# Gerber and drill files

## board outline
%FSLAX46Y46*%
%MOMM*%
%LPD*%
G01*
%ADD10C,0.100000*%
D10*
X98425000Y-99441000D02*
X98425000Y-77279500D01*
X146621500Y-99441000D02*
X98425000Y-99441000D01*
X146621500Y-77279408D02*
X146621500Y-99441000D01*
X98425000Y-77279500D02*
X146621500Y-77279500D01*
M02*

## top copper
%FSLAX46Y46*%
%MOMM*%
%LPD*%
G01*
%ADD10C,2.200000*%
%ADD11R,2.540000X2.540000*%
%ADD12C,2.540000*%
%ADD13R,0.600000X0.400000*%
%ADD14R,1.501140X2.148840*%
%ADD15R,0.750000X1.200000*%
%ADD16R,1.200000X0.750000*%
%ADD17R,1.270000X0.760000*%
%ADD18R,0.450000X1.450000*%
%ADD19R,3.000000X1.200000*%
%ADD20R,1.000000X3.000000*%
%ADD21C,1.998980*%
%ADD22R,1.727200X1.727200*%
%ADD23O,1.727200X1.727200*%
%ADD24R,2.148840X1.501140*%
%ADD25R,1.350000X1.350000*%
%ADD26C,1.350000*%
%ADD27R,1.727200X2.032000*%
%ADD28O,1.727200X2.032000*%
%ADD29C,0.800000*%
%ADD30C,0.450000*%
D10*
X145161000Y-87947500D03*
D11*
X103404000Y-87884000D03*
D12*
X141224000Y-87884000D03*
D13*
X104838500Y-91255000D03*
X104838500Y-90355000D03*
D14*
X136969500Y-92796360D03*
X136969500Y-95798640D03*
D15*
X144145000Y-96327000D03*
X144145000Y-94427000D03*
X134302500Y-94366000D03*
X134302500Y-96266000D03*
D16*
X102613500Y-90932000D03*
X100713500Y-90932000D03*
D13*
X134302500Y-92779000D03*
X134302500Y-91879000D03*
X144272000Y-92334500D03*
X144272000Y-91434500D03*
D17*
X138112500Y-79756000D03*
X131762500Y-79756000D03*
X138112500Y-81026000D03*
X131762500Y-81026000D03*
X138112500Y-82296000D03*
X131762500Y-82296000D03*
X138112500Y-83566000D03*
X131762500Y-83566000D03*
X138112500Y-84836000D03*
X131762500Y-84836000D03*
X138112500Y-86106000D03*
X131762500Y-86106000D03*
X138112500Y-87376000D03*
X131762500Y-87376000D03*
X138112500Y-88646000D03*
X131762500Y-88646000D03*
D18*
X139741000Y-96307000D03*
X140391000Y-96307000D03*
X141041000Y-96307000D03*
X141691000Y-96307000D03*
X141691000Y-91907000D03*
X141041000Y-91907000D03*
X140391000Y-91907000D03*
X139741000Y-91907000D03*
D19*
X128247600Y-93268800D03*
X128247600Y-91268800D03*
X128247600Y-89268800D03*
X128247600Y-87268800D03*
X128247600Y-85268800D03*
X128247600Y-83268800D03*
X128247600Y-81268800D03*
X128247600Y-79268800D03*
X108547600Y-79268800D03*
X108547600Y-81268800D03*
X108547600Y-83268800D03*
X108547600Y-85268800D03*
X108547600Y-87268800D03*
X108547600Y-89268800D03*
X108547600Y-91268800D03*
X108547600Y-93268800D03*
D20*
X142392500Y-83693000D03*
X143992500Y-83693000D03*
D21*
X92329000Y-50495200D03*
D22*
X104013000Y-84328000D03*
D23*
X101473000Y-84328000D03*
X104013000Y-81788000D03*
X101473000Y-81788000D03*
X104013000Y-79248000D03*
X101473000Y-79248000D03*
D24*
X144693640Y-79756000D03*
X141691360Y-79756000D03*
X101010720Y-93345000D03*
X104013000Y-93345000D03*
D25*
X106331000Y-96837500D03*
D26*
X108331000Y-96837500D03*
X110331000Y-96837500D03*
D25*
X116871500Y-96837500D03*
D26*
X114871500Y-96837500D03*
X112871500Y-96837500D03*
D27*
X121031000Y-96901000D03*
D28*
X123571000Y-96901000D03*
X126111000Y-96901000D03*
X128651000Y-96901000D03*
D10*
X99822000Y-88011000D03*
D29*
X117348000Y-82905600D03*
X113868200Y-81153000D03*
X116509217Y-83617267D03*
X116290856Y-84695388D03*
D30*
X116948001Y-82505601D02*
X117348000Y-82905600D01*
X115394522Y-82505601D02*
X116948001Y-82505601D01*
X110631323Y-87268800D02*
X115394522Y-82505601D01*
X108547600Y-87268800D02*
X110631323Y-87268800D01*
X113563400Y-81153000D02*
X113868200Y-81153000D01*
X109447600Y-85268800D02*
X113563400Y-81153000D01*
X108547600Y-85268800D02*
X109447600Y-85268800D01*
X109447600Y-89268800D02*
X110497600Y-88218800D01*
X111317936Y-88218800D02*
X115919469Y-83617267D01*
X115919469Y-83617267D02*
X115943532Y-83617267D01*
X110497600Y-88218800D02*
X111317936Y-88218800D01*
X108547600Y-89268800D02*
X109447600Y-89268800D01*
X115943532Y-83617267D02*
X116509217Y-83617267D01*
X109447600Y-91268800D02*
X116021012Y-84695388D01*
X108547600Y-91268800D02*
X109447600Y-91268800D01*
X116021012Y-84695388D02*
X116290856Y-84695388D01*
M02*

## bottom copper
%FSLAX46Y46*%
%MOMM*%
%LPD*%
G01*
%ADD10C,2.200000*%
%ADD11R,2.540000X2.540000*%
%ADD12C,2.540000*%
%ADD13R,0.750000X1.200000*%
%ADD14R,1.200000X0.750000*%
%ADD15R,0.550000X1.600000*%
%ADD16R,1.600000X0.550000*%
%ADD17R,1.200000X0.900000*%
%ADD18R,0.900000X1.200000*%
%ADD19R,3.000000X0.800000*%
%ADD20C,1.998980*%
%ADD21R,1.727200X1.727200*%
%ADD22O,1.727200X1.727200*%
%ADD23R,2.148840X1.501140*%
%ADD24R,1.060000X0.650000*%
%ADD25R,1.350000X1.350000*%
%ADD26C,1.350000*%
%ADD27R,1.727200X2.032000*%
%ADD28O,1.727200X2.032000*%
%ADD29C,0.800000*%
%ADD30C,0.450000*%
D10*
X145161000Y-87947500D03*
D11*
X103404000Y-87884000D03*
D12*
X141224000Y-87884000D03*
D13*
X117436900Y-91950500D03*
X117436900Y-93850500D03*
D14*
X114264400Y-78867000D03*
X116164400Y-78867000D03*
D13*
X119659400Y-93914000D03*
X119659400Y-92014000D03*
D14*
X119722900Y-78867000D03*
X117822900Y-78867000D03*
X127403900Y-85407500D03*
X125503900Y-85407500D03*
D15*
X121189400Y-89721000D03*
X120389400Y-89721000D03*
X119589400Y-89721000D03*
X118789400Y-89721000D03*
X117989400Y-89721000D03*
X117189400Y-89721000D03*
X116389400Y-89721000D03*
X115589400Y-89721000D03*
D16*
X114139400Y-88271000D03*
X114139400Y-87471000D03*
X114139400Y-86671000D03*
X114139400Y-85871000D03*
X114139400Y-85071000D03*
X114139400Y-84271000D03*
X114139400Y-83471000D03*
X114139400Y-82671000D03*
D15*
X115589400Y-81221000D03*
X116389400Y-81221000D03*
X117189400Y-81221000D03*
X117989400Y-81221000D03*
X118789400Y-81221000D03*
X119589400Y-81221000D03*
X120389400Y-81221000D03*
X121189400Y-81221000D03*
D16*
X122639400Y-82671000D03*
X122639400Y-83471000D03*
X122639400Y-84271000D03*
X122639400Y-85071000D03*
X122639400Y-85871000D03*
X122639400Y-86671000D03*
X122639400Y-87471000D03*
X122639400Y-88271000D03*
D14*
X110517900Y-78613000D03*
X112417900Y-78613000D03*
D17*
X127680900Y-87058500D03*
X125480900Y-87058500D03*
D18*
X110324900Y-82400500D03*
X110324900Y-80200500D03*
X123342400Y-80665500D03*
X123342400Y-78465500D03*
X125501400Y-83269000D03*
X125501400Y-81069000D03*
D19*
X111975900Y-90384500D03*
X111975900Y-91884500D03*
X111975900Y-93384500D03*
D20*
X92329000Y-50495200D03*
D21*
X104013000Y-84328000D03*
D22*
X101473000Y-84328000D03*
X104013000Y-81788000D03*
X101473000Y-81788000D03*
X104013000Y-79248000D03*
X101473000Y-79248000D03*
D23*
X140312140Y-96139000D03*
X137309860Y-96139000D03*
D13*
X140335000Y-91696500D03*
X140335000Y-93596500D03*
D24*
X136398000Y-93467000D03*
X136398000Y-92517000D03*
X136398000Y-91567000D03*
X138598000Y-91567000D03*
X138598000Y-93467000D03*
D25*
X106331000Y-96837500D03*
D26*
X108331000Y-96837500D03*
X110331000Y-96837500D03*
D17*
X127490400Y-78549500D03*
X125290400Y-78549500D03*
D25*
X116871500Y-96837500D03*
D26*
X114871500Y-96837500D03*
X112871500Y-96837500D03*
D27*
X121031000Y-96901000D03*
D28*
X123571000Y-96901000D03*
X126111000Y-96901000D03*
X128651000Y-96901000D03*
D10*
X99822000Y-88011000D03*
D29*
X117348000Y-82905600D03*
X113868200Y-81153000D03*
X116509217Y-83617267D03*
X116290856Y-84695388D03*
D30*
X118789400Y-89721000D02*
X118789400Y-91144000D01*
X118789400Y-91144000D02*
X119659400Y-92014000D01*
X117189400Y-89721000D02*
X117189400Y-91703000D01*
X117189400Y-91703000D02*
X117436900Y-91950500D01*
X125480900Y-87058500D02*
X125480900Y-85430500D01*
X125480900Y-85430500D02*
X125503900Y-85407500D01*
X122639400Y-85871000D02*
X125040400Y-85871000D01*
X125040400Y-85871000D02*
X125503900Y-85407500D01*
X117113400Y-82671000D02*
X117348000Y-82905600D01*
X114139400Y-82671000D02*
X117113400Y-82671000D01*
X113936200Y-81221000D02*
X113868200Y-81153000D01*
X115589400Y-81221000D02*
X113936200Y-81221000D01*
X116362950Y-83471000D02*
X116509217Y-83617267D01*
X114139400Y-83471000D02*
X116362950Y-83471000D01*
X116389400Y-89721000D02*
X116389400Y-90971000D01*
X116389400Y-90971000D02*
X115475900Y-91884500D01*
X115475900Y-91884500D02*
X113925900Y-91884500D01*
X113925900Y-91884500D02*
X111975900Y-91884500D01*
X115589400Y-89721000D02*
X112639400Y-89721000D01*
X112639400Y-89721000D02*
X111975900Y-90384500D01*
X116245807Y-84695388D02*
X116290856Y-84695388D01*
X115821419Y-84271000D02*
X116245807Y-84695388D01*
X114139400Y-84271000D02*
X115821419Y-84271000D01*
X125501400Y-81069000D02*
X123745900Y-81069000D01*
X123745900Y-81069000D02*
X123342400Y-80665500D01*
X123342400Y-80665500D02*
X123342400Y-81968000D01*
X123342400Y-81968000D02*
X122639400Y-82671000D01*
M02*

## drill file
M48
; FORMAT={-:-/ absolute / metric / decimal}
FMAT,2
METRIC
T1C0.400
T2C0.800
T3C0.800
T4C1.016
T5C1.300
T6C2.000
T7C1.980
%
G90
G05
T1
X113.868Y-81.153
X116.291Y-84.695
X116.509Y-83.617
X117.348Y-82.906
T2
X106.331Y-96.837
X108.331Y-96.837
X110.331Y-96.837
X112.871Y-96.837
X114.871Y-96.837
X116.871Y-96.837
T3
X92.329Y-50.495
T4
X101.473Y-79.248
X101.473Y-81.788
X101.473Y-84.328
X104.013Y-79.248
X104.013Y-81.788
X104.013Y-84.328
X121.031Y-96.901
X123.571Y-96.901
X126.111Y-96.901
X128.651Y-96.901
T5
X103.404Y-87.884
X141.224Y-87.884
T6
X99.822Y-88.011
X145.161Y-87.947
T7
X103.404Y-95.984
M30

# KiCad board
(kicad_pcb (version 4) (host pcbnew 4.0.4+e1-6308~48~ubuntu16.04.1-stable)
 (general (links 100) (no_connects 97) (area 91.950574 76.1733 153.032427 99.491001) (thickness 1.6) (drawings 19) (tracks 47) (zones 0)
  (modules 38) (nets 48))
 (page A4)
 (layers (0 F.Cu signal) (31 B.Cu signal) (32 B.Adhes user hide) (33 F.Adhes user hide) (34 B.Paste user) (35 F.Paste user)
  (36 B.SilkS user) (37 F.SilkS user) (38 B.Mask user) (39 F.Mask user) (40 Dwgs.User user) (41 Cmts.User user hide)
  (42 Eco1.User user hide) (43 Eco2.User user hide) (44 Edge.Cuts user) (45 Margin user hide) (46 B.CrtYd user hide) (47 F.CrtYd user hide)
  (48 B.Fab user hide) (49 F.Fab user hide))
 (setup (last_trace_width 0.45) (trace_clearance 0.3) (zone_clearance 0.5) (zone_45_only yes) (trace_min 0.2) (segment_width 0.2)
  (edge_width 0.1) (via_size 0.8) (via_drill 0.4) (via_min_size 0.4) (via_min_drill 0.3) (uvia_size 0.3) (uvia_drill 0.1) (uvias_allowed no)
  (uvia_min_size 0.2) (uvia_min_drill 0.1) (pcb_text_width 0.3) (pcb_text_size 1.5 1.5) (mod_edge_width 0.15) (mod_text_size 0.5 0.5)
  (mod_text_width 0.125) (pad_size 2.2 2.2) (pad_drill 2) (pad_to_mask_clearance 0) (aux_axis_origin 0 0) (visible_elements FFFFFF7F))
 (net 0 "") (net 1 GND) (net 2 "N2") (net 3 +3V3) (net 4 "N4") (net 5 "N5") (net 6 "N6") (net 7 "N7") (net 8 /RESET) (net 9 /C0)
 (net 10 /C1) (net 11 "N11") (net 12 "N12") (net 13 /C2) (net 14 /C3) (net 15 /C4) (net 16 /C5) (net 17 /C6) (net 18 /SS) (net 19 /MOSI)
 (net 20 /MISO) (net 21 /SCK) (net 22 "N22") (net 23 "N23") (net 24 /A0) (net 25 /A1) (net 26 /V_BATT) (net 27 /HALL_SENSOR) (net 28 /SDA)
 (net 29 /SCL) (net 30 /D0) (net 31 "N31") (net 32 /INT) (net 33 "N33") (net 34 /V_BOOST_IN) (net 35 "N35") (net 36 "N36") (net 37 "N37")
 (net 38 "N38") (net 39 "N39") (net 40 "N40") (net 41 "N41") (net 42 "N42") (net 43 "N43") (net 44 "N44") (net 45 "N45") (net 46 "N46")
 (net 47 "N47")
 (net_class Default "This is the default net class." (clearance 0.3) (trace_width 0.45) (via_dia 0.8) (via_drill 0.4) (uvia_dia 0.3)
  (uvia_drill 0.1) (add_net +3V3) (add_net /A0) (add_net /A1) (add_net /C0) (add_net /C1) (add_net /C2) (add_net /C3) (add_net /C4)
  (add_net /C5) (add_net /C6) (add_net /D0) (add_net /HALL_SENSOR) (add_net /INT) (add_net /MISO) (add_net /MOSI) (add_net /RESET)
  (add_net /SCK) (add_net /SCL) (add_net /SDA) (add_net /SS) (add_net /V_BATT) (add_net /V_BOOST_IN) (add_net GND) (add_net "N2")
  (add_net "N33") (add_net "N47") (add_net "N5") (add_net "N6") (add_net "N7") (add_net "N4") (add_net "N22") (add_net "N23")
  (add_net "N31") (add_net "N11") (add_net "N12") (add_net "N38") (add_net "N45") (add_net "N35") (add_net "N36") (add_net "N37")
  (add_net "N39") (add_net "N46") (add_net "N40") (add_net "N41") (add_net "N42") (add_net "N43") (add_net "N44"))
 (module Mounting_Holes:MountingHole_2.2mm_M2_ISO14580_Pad (layer F.Cu) (at 145.161 87.9475)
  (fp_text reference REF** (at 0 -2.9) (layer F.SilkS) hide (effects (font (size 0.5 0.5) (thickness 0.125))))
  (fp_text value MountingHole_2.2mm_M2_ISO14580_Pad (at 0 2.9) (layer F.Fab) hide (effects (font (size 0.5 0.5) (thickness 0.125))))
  (pad "" thru_hole circle (at 0 0) (size 2.2 2.2) (drill 2) (layers *.Cu *.Mask F.SilkS) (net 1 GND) (zone_connect 2)))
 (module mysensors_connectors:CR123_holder (layer B.Cu) (at 103.404 87.884 270)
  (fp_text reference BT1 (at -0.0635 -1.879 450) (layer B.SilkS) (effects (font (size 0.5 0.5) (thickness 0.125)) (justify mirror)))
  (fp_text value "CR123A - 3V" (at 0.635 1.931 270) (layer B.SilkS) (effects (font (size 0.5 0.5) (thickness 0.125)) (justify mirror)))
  (pad 1 thru_hole rect (at 0 0 270) (size 2.54 2.54) (drill 1.3) (layers *.Cu *.Mask B.SilkS) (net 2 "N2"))
  (pad 2 thru_hole circle (at 0 -37.82 270) (size 2.54 2.54) (drill 1.3) (layers *.Cu *.Mask B.SilkS) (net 1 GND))
  (pad "" np_thru_hole circle (at 8.1 0 270) (size 1.98 1.98) (drill 1.98) (layers *.Cu Dwgs.User)))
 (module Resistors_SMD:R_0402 (layer F.Cu) (at 104.8385 90.805 90)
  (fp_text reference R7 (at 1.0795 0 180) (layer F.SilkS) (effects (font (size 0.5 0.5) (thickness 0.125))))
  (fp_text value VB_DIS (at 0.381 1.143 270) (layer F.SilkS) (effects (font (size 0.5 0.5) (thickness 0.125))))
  (pad 1 smd rect (at -0.45 0 90) (size 0.4 0.6) (layers F.Cu F.Paste F.Mask) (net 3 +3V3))
  (pad 2 smd rect (at 0.45 0 90) (size 0.4 0.6) (layers F.Cu F.Paste F.Mask) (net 2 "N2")))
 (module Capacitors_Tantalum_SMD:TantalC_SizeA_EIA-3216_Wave (layer F.Cu) (at 136.9695 94.2975 90)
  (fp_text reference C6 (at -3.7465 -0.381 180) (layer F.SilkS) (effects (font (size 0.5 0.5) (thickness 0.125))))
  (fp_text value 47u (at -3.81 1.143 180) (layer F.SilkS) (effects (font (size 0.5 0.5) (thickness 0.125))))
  (pad 2 smd rect (at 1.50114 0 90) (size 2.14884 1.50114) (layers F.Cu F.Paste F.Mask) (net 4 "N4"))
  (pad 1 smd rect (at -1.50114 0 90) (size 2.14884 1.50114) (layers F.Cu F.Paste F.Mask) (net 1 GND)))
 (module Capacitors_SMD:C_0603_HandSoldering (layer B.Cu) (at 117.4369 92.9005 270)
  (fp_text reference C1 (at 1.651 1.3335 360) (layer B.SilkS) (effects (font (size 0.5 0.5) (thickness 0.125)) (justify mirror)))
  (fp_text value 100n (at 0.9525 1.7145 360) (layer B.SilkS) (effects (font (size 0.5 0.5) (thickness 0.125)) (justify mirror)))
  (pad 1 smd rect (at -0.95 0 270) (size 1.2 0.75) (layers B.Cu B.Paste B.Mask) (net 3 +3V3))
  (pad 2 smd rect (at 0.95 0 270) (size 1.2 0.75) (layers B.Cu B.Paste B.Mask) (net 1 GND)))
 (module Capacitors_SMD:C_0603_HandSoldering (layer B.Cu) (at 115.2144 78.867)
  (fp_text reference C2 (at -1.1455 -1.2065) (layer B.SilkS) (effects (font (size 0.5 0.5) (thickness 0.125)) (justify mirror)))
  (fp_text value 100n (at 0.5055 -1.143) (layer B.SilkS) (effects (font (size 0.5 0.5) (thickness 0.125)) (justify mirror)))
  (pad 1 smd rect (at -0.95 0) (size 1.2 0.75) (layers B.Cu B.Paste B.Mask) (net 1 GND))
  (pad 2 smd rect (at 0.95 0) (size 1.2 0.75) (layers B.Cu B.Paste B.Mask) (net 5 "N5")))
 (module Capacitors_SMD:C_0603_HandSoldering (layer B.Cu) (at 119.6594 92.964 90)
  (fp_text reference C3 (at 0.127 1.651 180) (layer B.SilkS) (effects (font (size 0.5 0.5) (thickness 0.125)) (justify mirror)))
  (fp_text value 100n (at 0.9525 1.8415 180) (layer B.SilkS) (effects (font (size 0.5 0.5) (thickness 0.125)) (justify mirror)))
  (pad 1 smd rect (at -0.95 0 90) (size 1.2 0.75) (layers B.Cu B.Paste B.Mask) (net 1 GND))
  (pad 2 smd rect (at 0.95 0 90) (size 1.2 0.75) (layers B.Cu B.Paste B.Mask) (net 3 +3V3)))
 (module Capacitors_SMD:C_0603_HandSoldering (layer B.Cu) (at 118.7729 78.867 180)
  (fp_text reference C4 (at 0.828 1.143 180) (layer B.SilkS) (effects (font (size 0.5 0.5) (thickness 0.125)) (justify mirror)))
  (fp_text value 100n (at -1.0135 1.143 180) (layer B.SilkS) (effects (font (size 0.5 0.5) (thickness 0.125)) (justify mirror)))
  (pad 1 smd rect (at -0.95 0 180) (size 1.2 0.75) (layers B.Cu B.Paste B.Mask) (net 1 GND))
  (pad 2 smd rect (at 0.95 0 180) (size 1.2 0.75) (layers B.Cu B.Paste B.Mask) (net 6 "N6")))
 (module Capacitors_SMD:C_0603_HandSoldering (layer F.Cu) (at 144.145 95.377 90)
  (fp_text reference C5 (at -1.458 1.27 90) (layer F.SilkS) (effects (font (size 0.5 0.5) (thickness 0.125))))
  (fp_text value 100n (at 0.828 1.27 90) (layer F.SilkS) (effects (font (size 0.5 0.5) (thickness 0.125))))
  (pad 1 smd rect (at -0.95 0 90) (size 1.2 0.75) (layers F.Cu F.Paste F.Mask) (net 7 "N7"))
  (pad 2 smd rect (at 0.95 0 90) (size 1.2 0.75) (layers F.Cu F.Paste F.Mask) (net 1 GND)))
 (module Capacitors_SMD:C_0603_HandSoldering (layer B.Cu) (at 126.4539 85.4075 180)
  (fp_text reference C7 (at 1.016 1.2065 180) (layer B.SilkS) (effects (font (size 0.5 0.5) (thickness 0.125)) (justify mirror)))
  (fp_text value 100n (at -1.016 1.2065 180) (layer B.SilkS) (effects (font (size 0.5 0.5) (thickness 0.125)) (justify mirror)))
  (pad 1 smd rect (at -0.95 0 180) (size 1.2 0.75) (layers B.Cu B.Paste B.Mask) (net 1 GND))
  (pad 2 smd rect (at 0.95 0 180) (size 1.2 0.75) (layers B.Cu B.Paste B.Mask) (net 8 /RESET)))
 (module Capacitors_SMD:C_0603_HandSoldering (layer F.Cu) (at 134.3025 95.316 270)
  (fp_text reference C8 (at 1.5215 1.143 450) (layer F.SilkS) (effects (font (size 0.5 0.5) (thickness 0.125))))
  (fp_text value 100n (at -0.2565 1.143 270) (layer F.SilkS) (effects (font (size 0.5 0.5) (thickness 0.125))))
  (pad 1 smd rect (at -0.95 0 270) (size 1.2 0.75) (layers F.Cu F.Paste F.Mask) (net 4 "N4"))
  (pad 2 smd rect (at 0.95 0 270) (size 1.2 0.75) (layers F.Cu F.Paste F.Mask) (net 1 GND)))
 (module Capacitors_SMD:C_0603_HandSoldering (layer F.Cu) (at 101.6635 90.932 180)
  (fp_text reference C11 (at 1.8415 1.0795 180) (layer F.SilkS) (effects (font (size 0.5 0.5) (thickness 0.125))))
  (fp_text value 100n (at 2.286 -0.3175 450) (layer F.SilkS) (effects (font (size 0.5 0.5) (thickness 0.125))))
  (pad 1 smd rect (at -0.95 0 180) (size 1.2 0.75) (layers F.Cu F.Paste F.Mask) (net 3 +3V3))
  (pad 2 smd rect (at 0.95 0 180) (size 1.2 0.75) (layers F.Cu F.Paste F.Mask) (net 1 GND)))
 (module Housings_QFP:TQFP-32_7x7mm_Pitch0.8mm (layer B.Cu) (at 118.3894 85.471 90)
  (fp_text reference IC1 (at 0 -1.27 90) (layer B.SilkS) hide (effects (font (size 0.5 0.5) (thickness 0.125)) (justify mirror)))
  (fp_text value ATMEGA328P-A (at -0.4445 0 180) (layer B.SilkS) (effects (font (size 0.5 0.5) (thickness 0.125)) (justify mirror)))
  (pad 1 smd rect (at -4.25 2.8 90) (size 1.6 0.55) (layers B.Cu B.Paste B.Mask) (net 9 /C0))
  (pad 2 smd rect (at -4.25 2 90) (size 1.6 0.55) (layers B.Cu B.Paste B.Mask) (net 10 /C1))
  (pad 3 smd rect (at -4.25 1.2 90) (size 1.6 0.55) (layers B.Cu B.Paste B.Mask) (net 1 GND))
  (pad 4 smd rect (at -4.25 0.4 90) (size 1.6 0.55) (layers B.Cu B.Paste B.Mask) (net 3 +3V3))
  (pad 5 smd rect (at -4.25 -0.4 90) (size 1.6 0.55) (layers B.Cu B.Paste B.Mask) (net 1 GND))
  (pad 6 smd rect (at -4.25 -1.2 90) (size 1.6 0.55) (layers B.Cu B.Paste B.Mask) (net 3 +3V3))
  (pad 7 smd rect (at -4.25 -2 90) (size 1.6 0.55) (layers B.Cu B.Paste B.Mask) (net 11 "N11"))
  (pad 8 smd rect (at -4.25 -2.8 90) (size 1.6 0.55) (layers B.Cu B.Paste B.Mask) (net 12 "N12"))
  (pad 9 smd rect (at -2.8 -4.25) (size 1.6 0.55) (layers B.Cu B.Paste B.Mask) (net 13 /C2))
  (pad 10 smd rect (at -2 -4.25) (size 1.6 0.55) (layers B.Cu B.Paste B.Mask) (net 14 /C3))
  (pad 11 smd rect (at -1.2 -4.25) (size 1.6 0.55) (layers B.Cu B.Paste B.Mask) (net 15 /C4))
  (pad 12 smd rect (at -0.4 -4.25) (size 1.6 0.55) (layers B.Cu B.Paste B.Mask) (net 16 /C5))
  (pad 13 smd rect (at 0.4 -4.25) (size 1.6 0.55) (layers B.Cu B.Paste B.Mask) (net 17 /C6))
  (pad 14 smd rect (at 1.2 -4.25) (size 1.6 0.55) (layers B.Cu B.Paste B.Mask) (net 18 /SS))
  (pad 15 smd rect (at 2 -4.25) (size 1.6 0.55) (layers B.Cu B.Paste B.Mask) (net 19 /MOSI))
  (pad 16 smd rect (at 2.8 -4.25) (size 1.6 0.55) (layers B.Cu B.Paste B.Mask) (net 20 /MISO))
  (pad 17 smd rect (at 4.25 -2.8 90) (size 1.6 0.55) (layers B.Cu B.Paste B.Mask) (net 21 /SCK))
  (pad 18 smd rect (at 4.25 -2 90) (size 1.6 0.55) (layers B.Cu B.Paste B.Mask) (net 5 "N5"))
  (pad 19 smd rect (at 4.25 -1.2 90) (size 1.6 0.55) (layers B.Cu B.Paste B.Mask) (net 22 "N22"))
  (pad 20 smd rect (at 4.25 -0.4 90) (size 1.6 0.55) (layers B.Cu B.Paste B.Mask) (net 6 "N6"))
  (pad 21 smd rect (at 4.25 0.4 90) (size 1.6 0.55) (layers B.Cu B.Paste B.Mask) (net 1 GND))
  (pad 22 smd rect (at 4.25 1.2 90) (size 1.6 0.55) (layers B.Cu B.Paste B.Mask) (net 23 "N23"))
  (pad 23 smd rect (at 4.25 2 90) (size 1.6 0.55) (layers B.Cu B.Paste B.Mask) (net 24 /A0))
  (pad 24 smd rect (at 4.25 2.8 90) (size 1.6 0.55) (layers B.Cu B.Paste B.Mask) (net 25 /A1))
  (pad 25 smd rect (at 2.8 4.25) (size 1.6 0.55) (layers B.Cu B.Paste B.Mask) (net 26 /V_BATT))
  (pad 26 smd rect (at 2 4.25) (size 1.6 0.55) (layers B.Cu B.Paste B.Mask) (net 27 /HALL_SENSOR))
  (pad 27 smd rect (at 1.2 4.25) (size 1.6 0.55) (layers B.Cu B.Paste B.Mask) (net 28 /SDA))
  (pad 28 smd rect (at 0.4 4.25) (size 1.6 0.55) (layers B.Cu B.Paste B.Mask) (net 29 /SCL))
  (pad 29 smd rect (at -0.4 4.25) (size 1.6 0.55) (layers B.Cu B.Paste B.Mask) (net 8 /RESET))
  (pad 30 smd rect (at -1.2 4.25) (size 1.6 0.55) (layers B.Cu B.Paste B.Mask) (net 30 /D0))
  (pad 31 smd rect (at -2 4.25) (size 1.6 0.55) (layers B.Cu B.Paste B.Mask) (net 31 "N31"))
  (pad 32 smd rect (at -2.8 4.25) (size 1.6 0.55) (layers B.Cu B.Paste B.Mask) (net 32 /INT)))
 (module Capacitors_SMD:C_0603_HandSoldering (layer B.Cu) (at 111.4679 78.613)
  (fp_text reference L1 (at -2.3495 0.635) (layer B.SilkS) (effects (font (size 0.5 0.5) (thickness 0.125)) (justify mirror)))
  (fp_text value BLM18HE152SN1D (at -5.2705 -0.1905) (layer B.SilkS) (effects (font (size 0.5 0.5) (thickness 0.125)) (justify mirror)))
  (pad 1 smd rect (at -0.95 0) (size 1.2 0.75) (layers B.Cu B.Paste B.Mask) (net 3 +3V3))
  (pad 2 smd rect (at 0.95 0) (size 1.2 0.75) (layers B.Cu B.Paste B.Mask) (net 5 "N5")))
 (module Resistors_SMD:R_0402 (layer F.Cu) (at 134.3025 92.329 90)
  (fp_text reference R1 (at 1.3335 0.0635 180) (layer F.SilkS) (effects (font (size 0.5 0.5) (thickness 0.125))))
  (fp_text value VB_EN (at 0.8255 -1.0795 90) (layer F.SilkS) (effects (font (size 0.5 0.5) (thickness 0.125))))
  (pad 1 smd rect (at -0.45 0 90) (size 0.4 0.6) (layers F.Cu F.Paste F.Mask) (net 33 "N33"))
  (pad 2 smd rect (at 0.45 0 90) (size 0.4 0.6) (layers F.Cu F.Paste F.Mask) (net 3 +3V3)))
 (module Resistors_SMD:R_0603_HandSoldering (layer B.Cu) (at 126.5809 87.0585 180)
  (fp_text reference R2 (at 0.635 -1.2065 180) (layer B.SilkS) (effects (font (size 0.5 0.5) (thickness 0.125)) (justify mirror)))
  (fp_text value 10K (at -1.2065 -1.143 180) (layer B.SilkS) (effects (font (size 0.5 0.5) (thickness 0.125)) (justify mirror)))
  (pad 1 smd rect (at -1.1 0 180) (size 1.2 0.9) (layers B.Cu B.Paste B.Mask) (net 3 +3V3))
  (pad 2 smd rect (at 1.1 0 180) (size 1.2 0.9) (layers B.Cu B.Paste B.Mask) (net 8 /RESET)))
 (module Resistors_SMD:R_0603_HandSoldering (layer B.Cu) (at 110.3249 81.3005 90)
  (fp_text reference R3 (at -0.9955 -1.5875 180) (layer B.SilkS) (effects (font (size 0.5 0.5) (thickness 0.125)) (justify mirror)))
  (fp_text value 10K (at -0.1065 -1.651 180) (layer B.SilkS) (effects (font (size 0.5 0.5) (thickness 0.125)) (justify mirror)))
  (pad 1 smd rect (at -1.1 0 90) (size 1.2 0.9) (layers B.Cu B.Paste B.Mask) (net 18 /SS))
  (pad 2 smd rect (at 1.1 0 90) (size 1.2 0.9) (layers B.Cu B.Paste B.Mask) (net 3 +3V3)))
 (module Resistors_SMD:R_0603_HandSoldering (layer B.Cu) (at 123.3424 79.5655 90)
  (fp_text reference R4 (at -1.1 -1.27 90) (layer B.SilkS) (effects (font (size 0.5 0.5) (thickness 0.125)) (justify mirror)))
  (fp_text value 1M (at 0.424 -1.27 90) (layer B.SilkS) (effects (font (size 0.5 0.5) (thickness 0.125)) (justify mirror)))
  (pad 1 smd rect (at -1.1 0 90) (size 1.2 0.9) (layers B.Cu B.Paste B.Mask) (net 26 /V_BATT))
  (pad 2 smd rect (at 1.1 0 90) (size 1.2 0.9) (layers B.Cu B.Paste B.Mask) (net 2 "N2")))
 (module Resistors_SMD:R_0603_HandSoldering (layer B.Cu) (at 125.5014 82.169 90)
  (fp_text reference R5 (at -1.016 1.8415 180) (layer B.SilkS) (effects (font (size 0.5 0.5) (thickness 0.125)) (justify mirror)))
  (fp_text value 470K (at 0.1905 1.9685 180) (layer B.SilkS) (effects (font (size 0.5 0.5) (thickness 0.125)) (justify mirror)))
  (pad 1 smd rect (at -1.1 0 90) (size 1.2 0.9) (layers B.Cu B.Paste B.Mask) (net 1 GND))
  (pad 2 smd rect (at 1.1 0 90) (size 1.2 0.9) (layers B.Cu B.Paste B.Mask) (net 26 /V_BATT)))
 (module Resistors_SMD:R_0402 (layer F.Cu) (at 144.272 91.8845 90)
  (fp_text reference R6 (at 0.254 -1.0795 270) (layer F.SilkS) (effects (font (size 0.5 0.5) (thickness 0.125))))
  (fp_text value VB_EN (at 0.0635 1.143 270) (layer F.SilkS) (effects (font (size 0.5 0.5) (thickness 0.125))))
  (pad 1 smd rect (at -0.45 0 90) (size 0.4 0.6) (layers F.Cu F.Paste F.Mask) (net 2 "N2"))
  (pad 2 smd rect (at 0.45 0 90) (size 0.4 0.6) (layers F.Cu F.Paste F.Mask) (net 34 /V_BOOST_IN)))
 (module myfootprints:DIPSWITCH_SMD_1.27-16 (layer F.Cu) (at 134.9375 84.201 270)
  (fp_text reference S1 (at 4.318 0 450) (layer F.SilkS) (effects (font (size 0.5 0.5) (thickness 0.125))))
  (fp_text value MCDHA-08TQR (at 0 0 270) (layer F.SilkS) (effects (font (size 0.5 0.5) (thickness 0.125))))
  (pad 16 smd rect (at -4.445 -3.175 270) (size 0.76 1.27) (layers F.Cu F.Paste F.Mask) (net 1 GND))
  (pad 1 smd rect (at -4.445 3.175 270) (size 0.76 1.27) (layers F.Cu F.Paste F.Mask) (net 9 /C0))
  (pad 15 smd rect (at -3.175 -3.175 270) (size 0.76 1.27) (layers F.Cu F.Paste F.Mask) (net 1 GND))
  (pad 2 smd rect (at -3.175 3.175 270) (size 0.76 1.27) (layers F.Cu F.Paste F.Mask) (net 10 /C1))
  (pad 14 smd rect (at -1.905 -3.175 270) (size 0.76 1.27) (layers F.Cu F.Paste F.Mask) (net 1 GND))
  (pad 3 smd rect (at -1.905 3.175 270) (size 0.76 1.27) (layers F.Cu F.Paste F.Mask) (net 13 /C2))
  (pad 13 smd rect (at -0.635 -3.175 270) (size 0.76 1.27) (layers F.Cu F.Paste F.Mask) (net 1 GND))
  (pad 4 smd rect (at -0.635 3.175 270) (size 0.76 1.27) (layers F.Cu F.Paste F.Mask) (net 14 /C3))
  (pad 12 smd rect (at 0.635 -3.175 270) (size 0.76 1.27) (layers F.Cu F.Paste F.Mask) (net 1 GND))
  (pad 5 smd rect (at 0.635 3.175 270) (size 0.76 1.27) (layers F.Cu F.Paste F.Mask) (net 15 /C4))
  (pad 11 smd rect (at 1.905 -3.175 270) (size 0.76 1.27) (layers F.Cu F.Paste F.Mask) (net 1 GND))
  (pad 6 smd rect (at 1.905 3.175 270) (size 0.76 1.27) (layers F.Cu F.Paste F.Mask) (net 16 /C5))
  (pad 10 smd rect (at 3.175 -3.175 270) (size 0.76 1.27) (layers F.Cu F.Paste F.Mask) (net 1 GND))
  (pad 7 smd rect (at 3.175 3.175 270) (size 0.76 1.27) (layers F.Cu F.Paste F.Mask) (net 17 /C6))
  (pad 9 smd rect (at 4.445 -3.175 270) (size 0.76 1.27) (layers F.Cu F.Paste F.Mask) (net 1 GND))
  (pad 8 smd rect (at 4.445 3.175 270) (size 0.76 1.27) (layers F.Cu F.Paste F.Mask) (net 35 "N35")))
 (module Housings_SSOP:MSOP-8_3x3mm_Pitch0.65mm (layer F.Cu) (at 140.716 94.107 90)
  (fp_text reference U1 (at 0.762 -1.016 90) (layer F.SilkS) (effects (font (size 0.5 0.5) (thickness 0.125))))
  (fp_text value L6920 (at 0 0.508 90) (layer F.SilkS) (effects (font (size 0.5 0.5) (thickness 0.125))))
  (pad 1 smd rect (at -2.2 -0.975 90) (size 1.45 0.45) (layers F.Cu F.Paste F.Mask) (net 4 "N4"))
  (pad 2 smd rect (at -2.2 -0.325 90) (size 1.45 0.45) (layers F.Cu F.Paste F.Mask) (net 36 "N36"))
  (pad 3 smd rect (at -2.2 0.325 90) (size 1.45 0.45) (layers F.Cu F.Paste F.Mask) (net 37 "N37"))
  (pad 4 smd rect (at -2.2 0.975 90) (size 1.45 0.45) (layers F.Cu F.Paste F.Mask) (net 7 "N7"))
  (pad 5 smd rect (at 2.2 0.975 90) (size 1.45 0.45) (layers F.Cu F.Paste F.Mask) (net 4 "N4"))
  (pad 6 smd rect (at 2.2 0.325 90) (size 1.45 0.45) (layers F.Cu F.Paste F.Mask) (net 1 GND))
  (pad 7 smd rect (at 2.2 -0.325 90) (size 1.45 0.45) (layers F.Cu F.Paste F.Mask) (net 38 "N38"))
  (pad 8 smd rect (at 2.2 -0.975 90) (size 1.45 0.45) (layers F.Cu F.Paste F.Mask) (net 4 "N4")))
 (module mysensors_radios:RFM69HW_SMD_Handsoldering (layer F.Cu) (at 126.8476 93.2688 180)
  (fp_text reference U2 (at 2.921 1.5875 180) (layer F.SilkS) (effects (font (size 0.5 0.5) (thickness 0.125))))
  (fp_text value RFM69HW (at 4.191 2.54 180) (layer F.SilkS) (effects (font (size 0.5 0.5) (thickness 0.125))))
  (pad 1 smd rect (at -1.4 0 180) (size 3 1.2) (layers F.Cu F.Paste F.Mask) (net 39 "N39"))
  (pad 2 smd rect (at -1.4 2 180) (size 3 1.2) (layers F.Cu F.Paste F.Mask) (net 32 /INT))
  (pad 3 smd rect (at -1.4 4 180) (size 3 1.2) (layers F.Cu F.Paste F.Mask) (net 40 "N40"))
  (pad 4 smd rect (at -1.4 6 180) (size 3 1.2) (layers F.Cu F.Paste F.Mask) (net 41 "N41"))
  (pad 5 smd rect (at -1.4 8 180) (size 3 1.2) (layers F.Cu F.Paste F.Mask) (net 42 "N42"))
  (pad 6 smd rect (at -1.4 10 180) (size 3 1.2) (layers F.Cu F.Paste F.Mask) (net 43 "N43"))
  (pad 7 smd rect (at -1.4 12 180) (size 3 1.2) (layers F.Cu F.Paste F.Mask) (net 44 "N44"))
  (pad 8 smd rect (at -1.4 14 180) (size 3 1.2) (layers F.Cu F.Paste F.Mask) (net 3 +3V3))
  (pad 9 smd rect (at 18.3 14 180) (size 3 1.2) (layers F.Cu F.Paste F.Mask) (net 1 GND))
  (pad 10 smd rect (at 18.3 12 180) (size 3 1.2) (layers F.Cu F.Paste F.Mask) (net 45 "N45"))
  (pad 11 smd rect (at 18.3 10 180) (size 3 1.2) (layers F.Cu F.Paste F.Mask) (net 1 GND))
  (pad 12 smd rect (at 18.3 8 180) (size 3 1.2) (layers F.Cu F.Paste F.Mask) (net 21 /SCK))
  (pad 13 smd rect (at 18.3 6 180) (size 3 1.2) (layers F.Cu F.Paste F.Mask) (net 20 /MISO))
  (pad 14 smd rect (at 18.3 4 180) (size 3 1.2) (layers F.Cu F.Paste F.Mask) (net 19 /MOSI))
  (pad 15 smd rect (at 18.3 2 180) (size 3 1.2) (layers F.Cu F.Paste F.Mask) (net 18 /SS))
  (pad 16 smd rect (at 18.3 0 180) (size 3 1.2) (layers F.Cu F.Paste F.Mask) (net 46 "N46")))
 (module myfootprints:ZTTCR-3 (layer B.Cu) (at 111.9759 91.8845 270)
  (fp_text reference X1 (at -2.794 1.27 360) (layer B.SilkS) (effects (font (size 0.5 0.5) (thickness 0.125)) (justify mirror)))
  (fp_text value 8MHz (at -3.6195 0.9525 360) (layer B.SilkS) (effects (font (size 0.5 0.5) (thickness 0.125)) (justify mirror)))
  (pad 1 smd rect (at -1.5 0 270) (size 0.8 3) (layers B.Cu B.Paste B.Mask) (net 12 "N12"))
  (pad 2 smd rect (at 0 0 270) (size 0.8 3) (layers B.Cu B.Paste B.Mask) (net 11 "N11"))
  (pad 3 smd rect (at 1.5 0 270) (size 0.8 3) (layers B.Cu B.Paste B.Mask) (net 1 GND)))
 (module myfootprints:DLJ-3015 (layer F.Cu) (at 143.1925 83.693)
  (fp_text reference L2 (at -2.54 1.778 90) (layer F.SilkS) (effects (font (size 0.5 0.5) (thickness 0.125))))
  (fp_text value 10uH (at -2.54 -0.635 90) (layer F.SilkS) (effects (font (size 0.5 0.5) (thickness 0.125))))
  (pad 1 smd rect (at -0.8 0) (size 1 3) (layers F.Cu F.Paste F.Mask) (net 38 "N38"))
  (pad 2 smd rect (at 0.8 0) (size 1 3) (layers F.Cu F.Paste F.Mask) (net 34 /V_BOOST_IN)))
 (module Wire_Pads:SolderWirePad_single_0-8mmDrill (layer F.Cu) (at 92.329 50.4952)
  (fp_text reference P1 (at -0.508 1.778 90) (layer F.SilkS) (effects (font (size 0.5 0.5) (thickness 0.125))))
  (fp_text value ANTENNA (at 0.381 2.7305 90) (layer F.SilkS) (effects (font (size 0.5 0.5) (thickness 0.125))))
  (pad 1 thru_hole circle (at 0 0) (size 1.99898 1.99898) (drill 0.8001) (layers *.Cu *.Mask F.SilkS) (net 45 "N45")))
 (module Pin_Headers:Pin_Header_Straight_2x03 (layer F.Cu) (at 104.013 84.328 180)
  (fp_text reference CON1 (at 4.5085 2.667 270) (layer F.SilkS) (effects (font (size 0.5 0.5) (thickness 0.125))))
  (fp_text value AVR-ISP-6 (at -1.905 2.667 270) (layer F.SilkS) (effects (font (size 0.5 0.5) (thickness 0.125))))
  (pad 1 thru_hole rect (at 0 0 180) (size 1.7272 1.7272) (drill 1.016) (layers *.Cu *.Mask F.SilkS) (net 20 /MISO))
  (pad 2 thru_hole oval (at 2.54 0 180) (size 1.7272 1.7272) (drill 1.016) (layers *.Cu *.Mask F.SilkS) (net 3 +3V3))
  (pad 3 thru_hole oval (at 0 2.54 180) (size 1.7272 1.7272) (drill 1.016) (layers *.Cu *.Mask F.SilkS) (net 21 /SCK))
  (pad 4 thru_hole oval (at 2.54 2.54 180) (size 1.7272 1.7272) (drill 1.016) (layers *.Cu *.Mask F.SilkS) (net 19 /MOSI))
  (pad 5 thru_hole oval (at 0 5.08 180) (size 1.7272 1.7272) (drill 1.016) (layers *.Cu *.Mask F.SilkS) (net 8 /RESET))
  (pad 6 thru_hole oval (at 2.54 5.08 180) (size 1.7272 1.7272) (drill 1.016) (layers *.Cu *.Mask F.SilkS) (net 1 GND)))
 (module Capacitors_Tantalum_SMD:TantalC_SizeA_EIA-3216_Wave (layer F.Cu) (at 143.1925 79.756)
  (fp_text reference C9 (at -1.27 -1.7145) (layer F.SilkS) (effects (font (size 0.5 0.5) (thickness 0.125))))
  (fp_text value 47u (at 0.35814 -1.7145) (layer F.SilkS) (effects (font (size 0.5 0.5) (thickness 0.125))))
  (pad 2 smd rect (at 1.50114 0) (size 2.14884 1.50114) (layers F.Cu F.Paste F.Mask) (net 34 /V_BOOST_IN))
  (pad 1 smd rect (at -1.50114 0) (size 2.14884 1.50114) (layers F.Cu F.Paste F.Mask) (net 1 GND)))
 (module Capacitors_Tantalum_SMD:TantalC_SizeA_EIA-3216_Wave (layer F.Cu) (at 102.51186 93.345 180)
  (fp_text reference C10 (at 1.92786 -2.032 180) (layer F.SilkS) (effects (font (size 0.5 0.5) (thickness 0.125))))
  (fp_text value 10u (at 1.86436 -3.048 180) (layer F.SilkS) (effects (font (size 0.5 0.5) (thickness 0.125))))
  (pad 2 smd rect (at 1.50114 0 180) (size 2.14884 1.50114) (layers F.Cu F.Paste F.Mask) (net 1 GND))
  (pad 1 smd rect (at -1.50114 0 180) (size 2.14884 1.50114) (layers F.Cu F.Paste F.Mask) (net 3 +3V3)))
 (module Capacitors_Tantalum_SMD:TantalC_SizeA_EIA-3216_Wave (layer B.Cu) (at 138.811 96.139)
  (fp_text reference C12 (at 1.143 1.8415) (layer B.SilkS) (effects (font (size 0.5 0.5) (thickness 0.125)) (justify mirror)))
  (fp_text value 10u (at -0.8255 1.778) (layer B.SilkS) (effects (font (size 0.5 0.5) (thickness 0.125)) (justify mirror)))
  (pad 2 smd rect (at 1.50114 0) (size 2.14884 1.50114) (layers B.Cu B.Paste B.Mask) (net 1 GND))
  (pad 1 smd rect (at -1.50114 0) (size 2.14884 1.50114) (layers B.Cu B.Paste B.Mask) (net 33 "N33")))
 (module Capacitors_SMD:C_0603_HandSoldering (layer B.Cu) (at 140.335 92.6465 270)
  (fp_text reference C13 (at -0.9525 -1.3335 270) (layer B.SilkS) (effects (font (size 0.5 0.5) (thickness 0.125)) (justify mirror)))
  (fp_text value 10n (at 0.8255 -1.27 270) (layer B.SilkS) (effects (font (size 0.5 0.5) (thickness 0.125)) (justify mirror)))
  (pad 1 smd rect (at -0.95 0 270) (size 1.2 0.75) (layers B.Cu B.Paste B.Mask) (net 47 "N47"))
  (pad 2 smd rect (at 0.95 0 270) (size 1.2 0.75) (layers B.Cu B.Paste B.Mask) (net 1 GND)))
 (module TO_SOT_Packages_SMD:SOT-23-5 (layer B.Cu) (at 137.498 92.517)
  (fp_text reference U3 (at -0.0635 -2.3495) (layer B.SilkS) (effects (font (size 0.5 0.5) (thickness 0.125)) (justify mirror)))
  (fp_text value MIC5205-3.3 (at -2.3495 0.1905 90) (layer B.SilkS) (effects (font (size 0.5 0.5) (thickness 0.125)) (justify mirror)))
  (pad 1 smd rect (at -1.1 0.95) (size 1.06 0.65) (layers B.Cu B.Paste B.Mask) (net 4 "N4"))
  (pad 2 smd rect (at -1.1 0) (size 1.06 0.65) (layers B.Cu B.Paste B.Mask) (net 1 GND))
  (pad 3 smd rect (at -1.1 -0.95) (size 1.06 0.65) (layers B.Cu B.Paste B.Mask) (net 4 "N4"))
  (pad 4 smd rect (at 1.1 -0.95) (size 1.06 0.65) (layers B.Cu B.Paste B.Mask) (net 47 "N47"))
  (pad 5 smd rect (at 1.1 0.95) (size 1.06 0.65) (layers B.Cu B.Paste B.Mask) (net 33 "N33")))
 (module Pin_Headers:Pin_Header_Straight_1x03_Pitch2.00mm (layer F.Cu) (at 106.331 96.8375 90)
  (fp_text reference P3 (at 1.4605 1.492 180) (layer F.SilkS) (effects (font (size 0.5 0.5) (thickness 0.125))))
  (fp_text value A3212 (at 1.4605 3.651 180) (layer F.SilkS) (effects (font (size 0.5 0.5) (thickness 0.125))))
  (pad 1 thru_hole rect (at 0 0 90) (size 1.35 1.35) (drill 0.8) (layers *.Cu *.Mask) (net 3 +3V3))
  (pad 2 thru_hole circle (at 0 2 90) (size 1.35 1.35) (drill 0.8) (layers *.Cu *.Mask) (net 1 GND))
  (pad 3 thru_hole circle (at 0 4 90) (size 1.35 1.35) (drill 0.8) (layers *.Cu *.Mask) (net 27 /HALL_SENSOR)))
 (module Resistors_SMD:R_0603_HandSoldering (layer B.Cu) (at 126.3904 78.5495 180)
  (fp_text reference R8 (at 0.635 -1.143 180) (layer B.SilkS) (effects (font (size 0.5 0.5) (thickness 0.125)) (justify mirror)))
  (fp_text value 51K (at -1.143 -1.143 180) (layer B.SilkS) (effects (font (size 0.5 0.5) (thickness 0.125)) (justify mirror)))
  (pad 1 smd rect (at -1.1 0 180) (size 1.2 0.9) (layers B.Cu B.Paste B.Mask) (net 3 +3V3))
  (pad 2 smd rect (at 1.1 0 180) (size 1.2 0.9) (layers B.Cu B.Paste B.Mask) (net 27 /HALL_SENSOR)))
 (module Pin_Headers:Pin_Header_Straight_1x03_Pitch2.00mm (layer F.Cu) (at 116.8715 96.8375 270)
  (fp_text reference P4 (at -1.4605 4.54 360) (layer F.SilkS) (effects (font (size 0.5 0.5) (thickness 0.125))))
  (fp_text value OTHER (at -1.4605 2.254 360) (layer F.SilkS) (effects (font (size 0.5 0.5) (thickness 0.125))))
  (pad 1 thru_hole rect (at 0 0 270) (size 1.35 1.35) (drill 0.8) (layers *.Cu *.Mask) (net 24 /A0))
  (pad 2 thru_hole circle (at 0 2 270) (size 1.35 1.35) (drill 0.8) (layers *.Cu *.Mask) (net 25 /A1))
  (pad 3 thru_hole circle (at 0 4 270) (size 1.35 1.35) (drill 0.8) (layers *.Cu *.Mask) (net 30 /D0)))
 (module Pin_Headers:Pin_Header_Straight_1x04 (layer F.Cu) (at 121.031 96.901 90)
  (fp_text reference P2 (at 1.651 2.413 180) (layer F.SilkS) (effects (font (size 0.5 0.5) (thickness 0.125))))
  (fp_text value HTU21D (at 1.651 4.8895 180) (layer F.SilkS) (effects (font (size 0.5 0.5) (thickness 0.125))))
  (pad 1 thru_hole rect (at 0 0 90) (size 2.032 1.7272) (drill 1.016) (layers *.Cu *.Mask F.SilkS) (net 3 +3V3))
  (pad 2 thru_hole oval (at 0 2.54 90) (size 2.032 1.7272) (drill 1.016) (layers *.Cu *.Mask F.SilkS) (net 1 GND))
  (pad 3 thru_hole oval (at 0 5.08 90) (size 2.032 1.7272) (drill 1.016) (layers *.Cu *.Mask F.SilkS) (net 28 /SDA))
  (pad 4 thru_hole oval (at 0 7.62 90) (size 2.032 1.7272) (drill 1.016) (layers *.Cu *.Mask F.SilkS) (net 29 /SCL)))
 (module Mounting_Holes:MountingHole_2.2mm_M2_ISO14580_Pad (layer F.Cu) (at 99.822 88.011)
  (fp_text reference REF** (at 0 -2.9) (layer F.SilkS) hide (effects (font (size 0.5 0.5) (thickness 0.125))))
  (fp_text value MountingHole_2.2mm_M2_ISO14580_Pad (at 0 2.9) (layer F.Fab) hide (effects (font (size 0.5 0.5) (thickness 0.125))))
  (pad "" thru_hole circle (at 0 0) (size 2.2 2.2) (drill 2) (layers *.Cu *.Mask F.SilkS) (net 1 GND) (zone_connect 2)))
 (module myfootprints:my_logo (layer B.Cu) (at 158.4706 77.8002)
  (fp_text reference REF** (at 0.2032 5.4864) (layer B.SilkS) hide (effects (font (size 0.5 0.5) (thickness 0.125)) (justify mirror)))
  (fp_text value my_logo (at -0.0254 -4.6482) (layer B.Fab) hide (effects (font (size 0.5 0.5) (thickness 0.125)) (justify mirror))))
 (gr_line (start 98.425 99.441) (end 98.425 77.2795) (layer Edge.Cuts) (width 0.1))
 (gr_line (start 146.6215 99.441) (end 98.425 99.441) (layer Edge.Cuts) (width 0.1))
 (gr_line (start 146.6215 77.279408) (end 146.6215 99.441) (layer Edge.Cuts) (width 0.1))
 (gr_line (start 98.425 77.2795) (end 146.6215 77.2795) (layer Edge.Cuts) (width 0.1))
 (segment (start 118.7894 89.721) (end 118.7894 91.144) (width 0.45) (layer B.Cu) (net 3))
 (segment (start 118.7894 91.144) (end 119.6594 92.014) (width 0.45) (layer B.Cu) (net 3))
 (segment (start 117.1894 89.721) (end 117.1894 91.703) (width 0.45) (layer B.Cu) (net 3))
 (segment (start 117.1894 91.703) (end 117.4369 91.9505) (width 0.45) (layer B.Cu) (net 3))
 (segment (start 125.4809 87.0585) (end 125.4809 85.4305) (width 0.45) (layer B.Cu) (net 8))
 (segment (start 125.4809 85.4305) (end 125.5039 85.4075) (width 0.45) (layer B.Cu) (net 8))
 (segment (start 122.6394 85.871) (end 125.0404 85.871) (width 0.45) (layer B.Cu) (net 8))
 (segment (start 125.0404 85.871) (end 125.5039 85.4075) (width 0.45) (layer B.Cu) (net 8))
 (segment (start 116.948001 82.505601) (end 117.348 82.9056) (width 0.45) (layer F.Cu) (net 20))
 (segment (start 117.1134 82.671) (end 117.348 82.9056) (width 0.45) (layer B.Cu) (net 20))
 (segment (start 114.1394 82.671) (end 117.1134 82.671) (width 0.45) (layer B.Cu) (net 20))
 (segment (start 115.394522 82.505601) (end 116.948001 82.505601) (width 0.45) (layer F.Cu) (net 20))
 (segment (start 110.631323 87.2688) (end 115.394522 82.505601) (width 0.45) (layer F.Cu) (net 20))
 (segment (start 108.5476 87.2688) (end 110.631323 87.2688) (width 0.45) (layer F.Cu) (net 20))
 (via (at 117.348 82.9056) (size 0.8) (drill 0.4) (layers F.Cu B.Cu) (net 20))
 (segment (start 113.5634 81.153) (end 113.8682 81.153) (width 0.45) (layer F.Cu) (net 21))
 (segment (start 109.4476 85.2688) (end 113.5634 81.153) (width 0.45) (layer F.Cu) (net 21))
 (segment (start 108.5476 85.2688) (end 109.4476 85.2688) (width 0.45) (layer F.Cu) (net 21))
 (segment (start 113.9362 81.221) (end 113.8682 81.153) (width 0.45) (layer B.Cu) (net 21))
 (segment (start 115.5894 81.221) (end 113.9362 81.221) (width 0.45) (layer B.Cu) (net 21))
 (via (at 113.8682 81.153) (size 0.8) (drill 0.4) (layers F.Cu B.Cu) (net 21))
 (segment (start 109.4476 89.2688) (end 110.4976 88.2188) (width 0.45) (layer F.Cu) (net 19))
 (segment (start 116.36295 83.471) (end 116.509217 83.617267) (width 0.45) (layer B.Cu) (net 19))
 (segment (start 111.317936 88.2188) (end 115.919469 83.617267) (width 0.45) (layer F.Cu) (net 19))
 (segment (start 115.919469 83.617267) (end 115.943532 83.617267) (width 0.45) (layer F.Cu) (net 19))
 (segment (start 110.4976 88.2188) (end 111.317936 88.2188) (width 0.45) (layer F.Cu) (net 19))
 (segment (start 108.5476 89.2688) (end 109.4476 89.2688) (width 0.45) (layer F.Cu) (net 19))
 (segment (start 115.943532 83.617267) (end 116.509217 83.617267) (width 0.45) (layer F.Cu) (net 19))
 (segment (start 114.1394 83.471) (end 116.36295 83.471) (width 0.45) (layer B.Cu) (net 19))
 (via (at 116.509217 83.617267) (size 0.8) (drill 0.4) (layers F.Cu B.Cu) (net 19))
 (segment (start 116.3894 89.721) (end 116.3894 90.971) (width 0.45) (layer B.Cu) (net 11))
 (segment (start 116.3894 90.971) (end 115.4759 91.8845) (width 0.45) (layer B.Cu) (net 11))
 (segment (start 115.4759 91.8845) (end 113.9259 91.8845) (width 0.45) (layer B.Cu) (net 11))
 (segment (start 113.9259 91.8845) (end 111.9759 91.8845) (width 0.45) (layer B.Cu) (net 11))
 (segment (start 115.5894 89.721) (end 112.6394 89.721) (width 0.45) (layer B.Cu) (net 12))
 (segment (start 112.6394 89.721) (end 111.9759 90.3845) (width 0.45) (layer B.Cu) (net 12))
 (segment (start 116.245807 84.695388) (end 116.290856 84.695388) (width 0.45) (layer B.Cu) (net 18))
 (segment (start 115.821419 84.271) (end 116.245807 84.695388) (width 0.45) (layer B.Cu) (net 18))
 (segment (start 109.4476 91.2688) (end 116.021012 84.695388) (width 0.45) (layer F.Cu) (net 18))
 (segment (start 108.5476 91.2688) (end 109.4476 91.2688) (width 0.45) (layer F.Cu) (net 18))
 (segment (start 116.021012 84.695388) (end 116.290856 84.695388) (width 0.45) (layer F.Cu) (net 18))
 (segment (start 114.1394 84.271) (end 115.821419 84.271) (width 0.45) (layer B.Cu) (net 18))
 (via (at 116.290856 84.695388) (size 0.8) (drill 0.4) (layers F.Cu B.Cu) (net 18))
 (segment (start 125.5014 81.069) (end 123.7459 81.069) (width 0.45) (layer B.Cu) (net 26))
 (segment (start 123.7459 81.069) (end 123.3424 80.6655) (width 0.45) (layer B.Cu) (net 26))
 (segment (start 123.3424 80.6655) (end 123.3424 81.968) (width 0.45) (layer B.Cu) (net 26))
 (segment (start 123.3424 81.968) (end 122.6394 82.671) (width 0.45) (layer B.Cu) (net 26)))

